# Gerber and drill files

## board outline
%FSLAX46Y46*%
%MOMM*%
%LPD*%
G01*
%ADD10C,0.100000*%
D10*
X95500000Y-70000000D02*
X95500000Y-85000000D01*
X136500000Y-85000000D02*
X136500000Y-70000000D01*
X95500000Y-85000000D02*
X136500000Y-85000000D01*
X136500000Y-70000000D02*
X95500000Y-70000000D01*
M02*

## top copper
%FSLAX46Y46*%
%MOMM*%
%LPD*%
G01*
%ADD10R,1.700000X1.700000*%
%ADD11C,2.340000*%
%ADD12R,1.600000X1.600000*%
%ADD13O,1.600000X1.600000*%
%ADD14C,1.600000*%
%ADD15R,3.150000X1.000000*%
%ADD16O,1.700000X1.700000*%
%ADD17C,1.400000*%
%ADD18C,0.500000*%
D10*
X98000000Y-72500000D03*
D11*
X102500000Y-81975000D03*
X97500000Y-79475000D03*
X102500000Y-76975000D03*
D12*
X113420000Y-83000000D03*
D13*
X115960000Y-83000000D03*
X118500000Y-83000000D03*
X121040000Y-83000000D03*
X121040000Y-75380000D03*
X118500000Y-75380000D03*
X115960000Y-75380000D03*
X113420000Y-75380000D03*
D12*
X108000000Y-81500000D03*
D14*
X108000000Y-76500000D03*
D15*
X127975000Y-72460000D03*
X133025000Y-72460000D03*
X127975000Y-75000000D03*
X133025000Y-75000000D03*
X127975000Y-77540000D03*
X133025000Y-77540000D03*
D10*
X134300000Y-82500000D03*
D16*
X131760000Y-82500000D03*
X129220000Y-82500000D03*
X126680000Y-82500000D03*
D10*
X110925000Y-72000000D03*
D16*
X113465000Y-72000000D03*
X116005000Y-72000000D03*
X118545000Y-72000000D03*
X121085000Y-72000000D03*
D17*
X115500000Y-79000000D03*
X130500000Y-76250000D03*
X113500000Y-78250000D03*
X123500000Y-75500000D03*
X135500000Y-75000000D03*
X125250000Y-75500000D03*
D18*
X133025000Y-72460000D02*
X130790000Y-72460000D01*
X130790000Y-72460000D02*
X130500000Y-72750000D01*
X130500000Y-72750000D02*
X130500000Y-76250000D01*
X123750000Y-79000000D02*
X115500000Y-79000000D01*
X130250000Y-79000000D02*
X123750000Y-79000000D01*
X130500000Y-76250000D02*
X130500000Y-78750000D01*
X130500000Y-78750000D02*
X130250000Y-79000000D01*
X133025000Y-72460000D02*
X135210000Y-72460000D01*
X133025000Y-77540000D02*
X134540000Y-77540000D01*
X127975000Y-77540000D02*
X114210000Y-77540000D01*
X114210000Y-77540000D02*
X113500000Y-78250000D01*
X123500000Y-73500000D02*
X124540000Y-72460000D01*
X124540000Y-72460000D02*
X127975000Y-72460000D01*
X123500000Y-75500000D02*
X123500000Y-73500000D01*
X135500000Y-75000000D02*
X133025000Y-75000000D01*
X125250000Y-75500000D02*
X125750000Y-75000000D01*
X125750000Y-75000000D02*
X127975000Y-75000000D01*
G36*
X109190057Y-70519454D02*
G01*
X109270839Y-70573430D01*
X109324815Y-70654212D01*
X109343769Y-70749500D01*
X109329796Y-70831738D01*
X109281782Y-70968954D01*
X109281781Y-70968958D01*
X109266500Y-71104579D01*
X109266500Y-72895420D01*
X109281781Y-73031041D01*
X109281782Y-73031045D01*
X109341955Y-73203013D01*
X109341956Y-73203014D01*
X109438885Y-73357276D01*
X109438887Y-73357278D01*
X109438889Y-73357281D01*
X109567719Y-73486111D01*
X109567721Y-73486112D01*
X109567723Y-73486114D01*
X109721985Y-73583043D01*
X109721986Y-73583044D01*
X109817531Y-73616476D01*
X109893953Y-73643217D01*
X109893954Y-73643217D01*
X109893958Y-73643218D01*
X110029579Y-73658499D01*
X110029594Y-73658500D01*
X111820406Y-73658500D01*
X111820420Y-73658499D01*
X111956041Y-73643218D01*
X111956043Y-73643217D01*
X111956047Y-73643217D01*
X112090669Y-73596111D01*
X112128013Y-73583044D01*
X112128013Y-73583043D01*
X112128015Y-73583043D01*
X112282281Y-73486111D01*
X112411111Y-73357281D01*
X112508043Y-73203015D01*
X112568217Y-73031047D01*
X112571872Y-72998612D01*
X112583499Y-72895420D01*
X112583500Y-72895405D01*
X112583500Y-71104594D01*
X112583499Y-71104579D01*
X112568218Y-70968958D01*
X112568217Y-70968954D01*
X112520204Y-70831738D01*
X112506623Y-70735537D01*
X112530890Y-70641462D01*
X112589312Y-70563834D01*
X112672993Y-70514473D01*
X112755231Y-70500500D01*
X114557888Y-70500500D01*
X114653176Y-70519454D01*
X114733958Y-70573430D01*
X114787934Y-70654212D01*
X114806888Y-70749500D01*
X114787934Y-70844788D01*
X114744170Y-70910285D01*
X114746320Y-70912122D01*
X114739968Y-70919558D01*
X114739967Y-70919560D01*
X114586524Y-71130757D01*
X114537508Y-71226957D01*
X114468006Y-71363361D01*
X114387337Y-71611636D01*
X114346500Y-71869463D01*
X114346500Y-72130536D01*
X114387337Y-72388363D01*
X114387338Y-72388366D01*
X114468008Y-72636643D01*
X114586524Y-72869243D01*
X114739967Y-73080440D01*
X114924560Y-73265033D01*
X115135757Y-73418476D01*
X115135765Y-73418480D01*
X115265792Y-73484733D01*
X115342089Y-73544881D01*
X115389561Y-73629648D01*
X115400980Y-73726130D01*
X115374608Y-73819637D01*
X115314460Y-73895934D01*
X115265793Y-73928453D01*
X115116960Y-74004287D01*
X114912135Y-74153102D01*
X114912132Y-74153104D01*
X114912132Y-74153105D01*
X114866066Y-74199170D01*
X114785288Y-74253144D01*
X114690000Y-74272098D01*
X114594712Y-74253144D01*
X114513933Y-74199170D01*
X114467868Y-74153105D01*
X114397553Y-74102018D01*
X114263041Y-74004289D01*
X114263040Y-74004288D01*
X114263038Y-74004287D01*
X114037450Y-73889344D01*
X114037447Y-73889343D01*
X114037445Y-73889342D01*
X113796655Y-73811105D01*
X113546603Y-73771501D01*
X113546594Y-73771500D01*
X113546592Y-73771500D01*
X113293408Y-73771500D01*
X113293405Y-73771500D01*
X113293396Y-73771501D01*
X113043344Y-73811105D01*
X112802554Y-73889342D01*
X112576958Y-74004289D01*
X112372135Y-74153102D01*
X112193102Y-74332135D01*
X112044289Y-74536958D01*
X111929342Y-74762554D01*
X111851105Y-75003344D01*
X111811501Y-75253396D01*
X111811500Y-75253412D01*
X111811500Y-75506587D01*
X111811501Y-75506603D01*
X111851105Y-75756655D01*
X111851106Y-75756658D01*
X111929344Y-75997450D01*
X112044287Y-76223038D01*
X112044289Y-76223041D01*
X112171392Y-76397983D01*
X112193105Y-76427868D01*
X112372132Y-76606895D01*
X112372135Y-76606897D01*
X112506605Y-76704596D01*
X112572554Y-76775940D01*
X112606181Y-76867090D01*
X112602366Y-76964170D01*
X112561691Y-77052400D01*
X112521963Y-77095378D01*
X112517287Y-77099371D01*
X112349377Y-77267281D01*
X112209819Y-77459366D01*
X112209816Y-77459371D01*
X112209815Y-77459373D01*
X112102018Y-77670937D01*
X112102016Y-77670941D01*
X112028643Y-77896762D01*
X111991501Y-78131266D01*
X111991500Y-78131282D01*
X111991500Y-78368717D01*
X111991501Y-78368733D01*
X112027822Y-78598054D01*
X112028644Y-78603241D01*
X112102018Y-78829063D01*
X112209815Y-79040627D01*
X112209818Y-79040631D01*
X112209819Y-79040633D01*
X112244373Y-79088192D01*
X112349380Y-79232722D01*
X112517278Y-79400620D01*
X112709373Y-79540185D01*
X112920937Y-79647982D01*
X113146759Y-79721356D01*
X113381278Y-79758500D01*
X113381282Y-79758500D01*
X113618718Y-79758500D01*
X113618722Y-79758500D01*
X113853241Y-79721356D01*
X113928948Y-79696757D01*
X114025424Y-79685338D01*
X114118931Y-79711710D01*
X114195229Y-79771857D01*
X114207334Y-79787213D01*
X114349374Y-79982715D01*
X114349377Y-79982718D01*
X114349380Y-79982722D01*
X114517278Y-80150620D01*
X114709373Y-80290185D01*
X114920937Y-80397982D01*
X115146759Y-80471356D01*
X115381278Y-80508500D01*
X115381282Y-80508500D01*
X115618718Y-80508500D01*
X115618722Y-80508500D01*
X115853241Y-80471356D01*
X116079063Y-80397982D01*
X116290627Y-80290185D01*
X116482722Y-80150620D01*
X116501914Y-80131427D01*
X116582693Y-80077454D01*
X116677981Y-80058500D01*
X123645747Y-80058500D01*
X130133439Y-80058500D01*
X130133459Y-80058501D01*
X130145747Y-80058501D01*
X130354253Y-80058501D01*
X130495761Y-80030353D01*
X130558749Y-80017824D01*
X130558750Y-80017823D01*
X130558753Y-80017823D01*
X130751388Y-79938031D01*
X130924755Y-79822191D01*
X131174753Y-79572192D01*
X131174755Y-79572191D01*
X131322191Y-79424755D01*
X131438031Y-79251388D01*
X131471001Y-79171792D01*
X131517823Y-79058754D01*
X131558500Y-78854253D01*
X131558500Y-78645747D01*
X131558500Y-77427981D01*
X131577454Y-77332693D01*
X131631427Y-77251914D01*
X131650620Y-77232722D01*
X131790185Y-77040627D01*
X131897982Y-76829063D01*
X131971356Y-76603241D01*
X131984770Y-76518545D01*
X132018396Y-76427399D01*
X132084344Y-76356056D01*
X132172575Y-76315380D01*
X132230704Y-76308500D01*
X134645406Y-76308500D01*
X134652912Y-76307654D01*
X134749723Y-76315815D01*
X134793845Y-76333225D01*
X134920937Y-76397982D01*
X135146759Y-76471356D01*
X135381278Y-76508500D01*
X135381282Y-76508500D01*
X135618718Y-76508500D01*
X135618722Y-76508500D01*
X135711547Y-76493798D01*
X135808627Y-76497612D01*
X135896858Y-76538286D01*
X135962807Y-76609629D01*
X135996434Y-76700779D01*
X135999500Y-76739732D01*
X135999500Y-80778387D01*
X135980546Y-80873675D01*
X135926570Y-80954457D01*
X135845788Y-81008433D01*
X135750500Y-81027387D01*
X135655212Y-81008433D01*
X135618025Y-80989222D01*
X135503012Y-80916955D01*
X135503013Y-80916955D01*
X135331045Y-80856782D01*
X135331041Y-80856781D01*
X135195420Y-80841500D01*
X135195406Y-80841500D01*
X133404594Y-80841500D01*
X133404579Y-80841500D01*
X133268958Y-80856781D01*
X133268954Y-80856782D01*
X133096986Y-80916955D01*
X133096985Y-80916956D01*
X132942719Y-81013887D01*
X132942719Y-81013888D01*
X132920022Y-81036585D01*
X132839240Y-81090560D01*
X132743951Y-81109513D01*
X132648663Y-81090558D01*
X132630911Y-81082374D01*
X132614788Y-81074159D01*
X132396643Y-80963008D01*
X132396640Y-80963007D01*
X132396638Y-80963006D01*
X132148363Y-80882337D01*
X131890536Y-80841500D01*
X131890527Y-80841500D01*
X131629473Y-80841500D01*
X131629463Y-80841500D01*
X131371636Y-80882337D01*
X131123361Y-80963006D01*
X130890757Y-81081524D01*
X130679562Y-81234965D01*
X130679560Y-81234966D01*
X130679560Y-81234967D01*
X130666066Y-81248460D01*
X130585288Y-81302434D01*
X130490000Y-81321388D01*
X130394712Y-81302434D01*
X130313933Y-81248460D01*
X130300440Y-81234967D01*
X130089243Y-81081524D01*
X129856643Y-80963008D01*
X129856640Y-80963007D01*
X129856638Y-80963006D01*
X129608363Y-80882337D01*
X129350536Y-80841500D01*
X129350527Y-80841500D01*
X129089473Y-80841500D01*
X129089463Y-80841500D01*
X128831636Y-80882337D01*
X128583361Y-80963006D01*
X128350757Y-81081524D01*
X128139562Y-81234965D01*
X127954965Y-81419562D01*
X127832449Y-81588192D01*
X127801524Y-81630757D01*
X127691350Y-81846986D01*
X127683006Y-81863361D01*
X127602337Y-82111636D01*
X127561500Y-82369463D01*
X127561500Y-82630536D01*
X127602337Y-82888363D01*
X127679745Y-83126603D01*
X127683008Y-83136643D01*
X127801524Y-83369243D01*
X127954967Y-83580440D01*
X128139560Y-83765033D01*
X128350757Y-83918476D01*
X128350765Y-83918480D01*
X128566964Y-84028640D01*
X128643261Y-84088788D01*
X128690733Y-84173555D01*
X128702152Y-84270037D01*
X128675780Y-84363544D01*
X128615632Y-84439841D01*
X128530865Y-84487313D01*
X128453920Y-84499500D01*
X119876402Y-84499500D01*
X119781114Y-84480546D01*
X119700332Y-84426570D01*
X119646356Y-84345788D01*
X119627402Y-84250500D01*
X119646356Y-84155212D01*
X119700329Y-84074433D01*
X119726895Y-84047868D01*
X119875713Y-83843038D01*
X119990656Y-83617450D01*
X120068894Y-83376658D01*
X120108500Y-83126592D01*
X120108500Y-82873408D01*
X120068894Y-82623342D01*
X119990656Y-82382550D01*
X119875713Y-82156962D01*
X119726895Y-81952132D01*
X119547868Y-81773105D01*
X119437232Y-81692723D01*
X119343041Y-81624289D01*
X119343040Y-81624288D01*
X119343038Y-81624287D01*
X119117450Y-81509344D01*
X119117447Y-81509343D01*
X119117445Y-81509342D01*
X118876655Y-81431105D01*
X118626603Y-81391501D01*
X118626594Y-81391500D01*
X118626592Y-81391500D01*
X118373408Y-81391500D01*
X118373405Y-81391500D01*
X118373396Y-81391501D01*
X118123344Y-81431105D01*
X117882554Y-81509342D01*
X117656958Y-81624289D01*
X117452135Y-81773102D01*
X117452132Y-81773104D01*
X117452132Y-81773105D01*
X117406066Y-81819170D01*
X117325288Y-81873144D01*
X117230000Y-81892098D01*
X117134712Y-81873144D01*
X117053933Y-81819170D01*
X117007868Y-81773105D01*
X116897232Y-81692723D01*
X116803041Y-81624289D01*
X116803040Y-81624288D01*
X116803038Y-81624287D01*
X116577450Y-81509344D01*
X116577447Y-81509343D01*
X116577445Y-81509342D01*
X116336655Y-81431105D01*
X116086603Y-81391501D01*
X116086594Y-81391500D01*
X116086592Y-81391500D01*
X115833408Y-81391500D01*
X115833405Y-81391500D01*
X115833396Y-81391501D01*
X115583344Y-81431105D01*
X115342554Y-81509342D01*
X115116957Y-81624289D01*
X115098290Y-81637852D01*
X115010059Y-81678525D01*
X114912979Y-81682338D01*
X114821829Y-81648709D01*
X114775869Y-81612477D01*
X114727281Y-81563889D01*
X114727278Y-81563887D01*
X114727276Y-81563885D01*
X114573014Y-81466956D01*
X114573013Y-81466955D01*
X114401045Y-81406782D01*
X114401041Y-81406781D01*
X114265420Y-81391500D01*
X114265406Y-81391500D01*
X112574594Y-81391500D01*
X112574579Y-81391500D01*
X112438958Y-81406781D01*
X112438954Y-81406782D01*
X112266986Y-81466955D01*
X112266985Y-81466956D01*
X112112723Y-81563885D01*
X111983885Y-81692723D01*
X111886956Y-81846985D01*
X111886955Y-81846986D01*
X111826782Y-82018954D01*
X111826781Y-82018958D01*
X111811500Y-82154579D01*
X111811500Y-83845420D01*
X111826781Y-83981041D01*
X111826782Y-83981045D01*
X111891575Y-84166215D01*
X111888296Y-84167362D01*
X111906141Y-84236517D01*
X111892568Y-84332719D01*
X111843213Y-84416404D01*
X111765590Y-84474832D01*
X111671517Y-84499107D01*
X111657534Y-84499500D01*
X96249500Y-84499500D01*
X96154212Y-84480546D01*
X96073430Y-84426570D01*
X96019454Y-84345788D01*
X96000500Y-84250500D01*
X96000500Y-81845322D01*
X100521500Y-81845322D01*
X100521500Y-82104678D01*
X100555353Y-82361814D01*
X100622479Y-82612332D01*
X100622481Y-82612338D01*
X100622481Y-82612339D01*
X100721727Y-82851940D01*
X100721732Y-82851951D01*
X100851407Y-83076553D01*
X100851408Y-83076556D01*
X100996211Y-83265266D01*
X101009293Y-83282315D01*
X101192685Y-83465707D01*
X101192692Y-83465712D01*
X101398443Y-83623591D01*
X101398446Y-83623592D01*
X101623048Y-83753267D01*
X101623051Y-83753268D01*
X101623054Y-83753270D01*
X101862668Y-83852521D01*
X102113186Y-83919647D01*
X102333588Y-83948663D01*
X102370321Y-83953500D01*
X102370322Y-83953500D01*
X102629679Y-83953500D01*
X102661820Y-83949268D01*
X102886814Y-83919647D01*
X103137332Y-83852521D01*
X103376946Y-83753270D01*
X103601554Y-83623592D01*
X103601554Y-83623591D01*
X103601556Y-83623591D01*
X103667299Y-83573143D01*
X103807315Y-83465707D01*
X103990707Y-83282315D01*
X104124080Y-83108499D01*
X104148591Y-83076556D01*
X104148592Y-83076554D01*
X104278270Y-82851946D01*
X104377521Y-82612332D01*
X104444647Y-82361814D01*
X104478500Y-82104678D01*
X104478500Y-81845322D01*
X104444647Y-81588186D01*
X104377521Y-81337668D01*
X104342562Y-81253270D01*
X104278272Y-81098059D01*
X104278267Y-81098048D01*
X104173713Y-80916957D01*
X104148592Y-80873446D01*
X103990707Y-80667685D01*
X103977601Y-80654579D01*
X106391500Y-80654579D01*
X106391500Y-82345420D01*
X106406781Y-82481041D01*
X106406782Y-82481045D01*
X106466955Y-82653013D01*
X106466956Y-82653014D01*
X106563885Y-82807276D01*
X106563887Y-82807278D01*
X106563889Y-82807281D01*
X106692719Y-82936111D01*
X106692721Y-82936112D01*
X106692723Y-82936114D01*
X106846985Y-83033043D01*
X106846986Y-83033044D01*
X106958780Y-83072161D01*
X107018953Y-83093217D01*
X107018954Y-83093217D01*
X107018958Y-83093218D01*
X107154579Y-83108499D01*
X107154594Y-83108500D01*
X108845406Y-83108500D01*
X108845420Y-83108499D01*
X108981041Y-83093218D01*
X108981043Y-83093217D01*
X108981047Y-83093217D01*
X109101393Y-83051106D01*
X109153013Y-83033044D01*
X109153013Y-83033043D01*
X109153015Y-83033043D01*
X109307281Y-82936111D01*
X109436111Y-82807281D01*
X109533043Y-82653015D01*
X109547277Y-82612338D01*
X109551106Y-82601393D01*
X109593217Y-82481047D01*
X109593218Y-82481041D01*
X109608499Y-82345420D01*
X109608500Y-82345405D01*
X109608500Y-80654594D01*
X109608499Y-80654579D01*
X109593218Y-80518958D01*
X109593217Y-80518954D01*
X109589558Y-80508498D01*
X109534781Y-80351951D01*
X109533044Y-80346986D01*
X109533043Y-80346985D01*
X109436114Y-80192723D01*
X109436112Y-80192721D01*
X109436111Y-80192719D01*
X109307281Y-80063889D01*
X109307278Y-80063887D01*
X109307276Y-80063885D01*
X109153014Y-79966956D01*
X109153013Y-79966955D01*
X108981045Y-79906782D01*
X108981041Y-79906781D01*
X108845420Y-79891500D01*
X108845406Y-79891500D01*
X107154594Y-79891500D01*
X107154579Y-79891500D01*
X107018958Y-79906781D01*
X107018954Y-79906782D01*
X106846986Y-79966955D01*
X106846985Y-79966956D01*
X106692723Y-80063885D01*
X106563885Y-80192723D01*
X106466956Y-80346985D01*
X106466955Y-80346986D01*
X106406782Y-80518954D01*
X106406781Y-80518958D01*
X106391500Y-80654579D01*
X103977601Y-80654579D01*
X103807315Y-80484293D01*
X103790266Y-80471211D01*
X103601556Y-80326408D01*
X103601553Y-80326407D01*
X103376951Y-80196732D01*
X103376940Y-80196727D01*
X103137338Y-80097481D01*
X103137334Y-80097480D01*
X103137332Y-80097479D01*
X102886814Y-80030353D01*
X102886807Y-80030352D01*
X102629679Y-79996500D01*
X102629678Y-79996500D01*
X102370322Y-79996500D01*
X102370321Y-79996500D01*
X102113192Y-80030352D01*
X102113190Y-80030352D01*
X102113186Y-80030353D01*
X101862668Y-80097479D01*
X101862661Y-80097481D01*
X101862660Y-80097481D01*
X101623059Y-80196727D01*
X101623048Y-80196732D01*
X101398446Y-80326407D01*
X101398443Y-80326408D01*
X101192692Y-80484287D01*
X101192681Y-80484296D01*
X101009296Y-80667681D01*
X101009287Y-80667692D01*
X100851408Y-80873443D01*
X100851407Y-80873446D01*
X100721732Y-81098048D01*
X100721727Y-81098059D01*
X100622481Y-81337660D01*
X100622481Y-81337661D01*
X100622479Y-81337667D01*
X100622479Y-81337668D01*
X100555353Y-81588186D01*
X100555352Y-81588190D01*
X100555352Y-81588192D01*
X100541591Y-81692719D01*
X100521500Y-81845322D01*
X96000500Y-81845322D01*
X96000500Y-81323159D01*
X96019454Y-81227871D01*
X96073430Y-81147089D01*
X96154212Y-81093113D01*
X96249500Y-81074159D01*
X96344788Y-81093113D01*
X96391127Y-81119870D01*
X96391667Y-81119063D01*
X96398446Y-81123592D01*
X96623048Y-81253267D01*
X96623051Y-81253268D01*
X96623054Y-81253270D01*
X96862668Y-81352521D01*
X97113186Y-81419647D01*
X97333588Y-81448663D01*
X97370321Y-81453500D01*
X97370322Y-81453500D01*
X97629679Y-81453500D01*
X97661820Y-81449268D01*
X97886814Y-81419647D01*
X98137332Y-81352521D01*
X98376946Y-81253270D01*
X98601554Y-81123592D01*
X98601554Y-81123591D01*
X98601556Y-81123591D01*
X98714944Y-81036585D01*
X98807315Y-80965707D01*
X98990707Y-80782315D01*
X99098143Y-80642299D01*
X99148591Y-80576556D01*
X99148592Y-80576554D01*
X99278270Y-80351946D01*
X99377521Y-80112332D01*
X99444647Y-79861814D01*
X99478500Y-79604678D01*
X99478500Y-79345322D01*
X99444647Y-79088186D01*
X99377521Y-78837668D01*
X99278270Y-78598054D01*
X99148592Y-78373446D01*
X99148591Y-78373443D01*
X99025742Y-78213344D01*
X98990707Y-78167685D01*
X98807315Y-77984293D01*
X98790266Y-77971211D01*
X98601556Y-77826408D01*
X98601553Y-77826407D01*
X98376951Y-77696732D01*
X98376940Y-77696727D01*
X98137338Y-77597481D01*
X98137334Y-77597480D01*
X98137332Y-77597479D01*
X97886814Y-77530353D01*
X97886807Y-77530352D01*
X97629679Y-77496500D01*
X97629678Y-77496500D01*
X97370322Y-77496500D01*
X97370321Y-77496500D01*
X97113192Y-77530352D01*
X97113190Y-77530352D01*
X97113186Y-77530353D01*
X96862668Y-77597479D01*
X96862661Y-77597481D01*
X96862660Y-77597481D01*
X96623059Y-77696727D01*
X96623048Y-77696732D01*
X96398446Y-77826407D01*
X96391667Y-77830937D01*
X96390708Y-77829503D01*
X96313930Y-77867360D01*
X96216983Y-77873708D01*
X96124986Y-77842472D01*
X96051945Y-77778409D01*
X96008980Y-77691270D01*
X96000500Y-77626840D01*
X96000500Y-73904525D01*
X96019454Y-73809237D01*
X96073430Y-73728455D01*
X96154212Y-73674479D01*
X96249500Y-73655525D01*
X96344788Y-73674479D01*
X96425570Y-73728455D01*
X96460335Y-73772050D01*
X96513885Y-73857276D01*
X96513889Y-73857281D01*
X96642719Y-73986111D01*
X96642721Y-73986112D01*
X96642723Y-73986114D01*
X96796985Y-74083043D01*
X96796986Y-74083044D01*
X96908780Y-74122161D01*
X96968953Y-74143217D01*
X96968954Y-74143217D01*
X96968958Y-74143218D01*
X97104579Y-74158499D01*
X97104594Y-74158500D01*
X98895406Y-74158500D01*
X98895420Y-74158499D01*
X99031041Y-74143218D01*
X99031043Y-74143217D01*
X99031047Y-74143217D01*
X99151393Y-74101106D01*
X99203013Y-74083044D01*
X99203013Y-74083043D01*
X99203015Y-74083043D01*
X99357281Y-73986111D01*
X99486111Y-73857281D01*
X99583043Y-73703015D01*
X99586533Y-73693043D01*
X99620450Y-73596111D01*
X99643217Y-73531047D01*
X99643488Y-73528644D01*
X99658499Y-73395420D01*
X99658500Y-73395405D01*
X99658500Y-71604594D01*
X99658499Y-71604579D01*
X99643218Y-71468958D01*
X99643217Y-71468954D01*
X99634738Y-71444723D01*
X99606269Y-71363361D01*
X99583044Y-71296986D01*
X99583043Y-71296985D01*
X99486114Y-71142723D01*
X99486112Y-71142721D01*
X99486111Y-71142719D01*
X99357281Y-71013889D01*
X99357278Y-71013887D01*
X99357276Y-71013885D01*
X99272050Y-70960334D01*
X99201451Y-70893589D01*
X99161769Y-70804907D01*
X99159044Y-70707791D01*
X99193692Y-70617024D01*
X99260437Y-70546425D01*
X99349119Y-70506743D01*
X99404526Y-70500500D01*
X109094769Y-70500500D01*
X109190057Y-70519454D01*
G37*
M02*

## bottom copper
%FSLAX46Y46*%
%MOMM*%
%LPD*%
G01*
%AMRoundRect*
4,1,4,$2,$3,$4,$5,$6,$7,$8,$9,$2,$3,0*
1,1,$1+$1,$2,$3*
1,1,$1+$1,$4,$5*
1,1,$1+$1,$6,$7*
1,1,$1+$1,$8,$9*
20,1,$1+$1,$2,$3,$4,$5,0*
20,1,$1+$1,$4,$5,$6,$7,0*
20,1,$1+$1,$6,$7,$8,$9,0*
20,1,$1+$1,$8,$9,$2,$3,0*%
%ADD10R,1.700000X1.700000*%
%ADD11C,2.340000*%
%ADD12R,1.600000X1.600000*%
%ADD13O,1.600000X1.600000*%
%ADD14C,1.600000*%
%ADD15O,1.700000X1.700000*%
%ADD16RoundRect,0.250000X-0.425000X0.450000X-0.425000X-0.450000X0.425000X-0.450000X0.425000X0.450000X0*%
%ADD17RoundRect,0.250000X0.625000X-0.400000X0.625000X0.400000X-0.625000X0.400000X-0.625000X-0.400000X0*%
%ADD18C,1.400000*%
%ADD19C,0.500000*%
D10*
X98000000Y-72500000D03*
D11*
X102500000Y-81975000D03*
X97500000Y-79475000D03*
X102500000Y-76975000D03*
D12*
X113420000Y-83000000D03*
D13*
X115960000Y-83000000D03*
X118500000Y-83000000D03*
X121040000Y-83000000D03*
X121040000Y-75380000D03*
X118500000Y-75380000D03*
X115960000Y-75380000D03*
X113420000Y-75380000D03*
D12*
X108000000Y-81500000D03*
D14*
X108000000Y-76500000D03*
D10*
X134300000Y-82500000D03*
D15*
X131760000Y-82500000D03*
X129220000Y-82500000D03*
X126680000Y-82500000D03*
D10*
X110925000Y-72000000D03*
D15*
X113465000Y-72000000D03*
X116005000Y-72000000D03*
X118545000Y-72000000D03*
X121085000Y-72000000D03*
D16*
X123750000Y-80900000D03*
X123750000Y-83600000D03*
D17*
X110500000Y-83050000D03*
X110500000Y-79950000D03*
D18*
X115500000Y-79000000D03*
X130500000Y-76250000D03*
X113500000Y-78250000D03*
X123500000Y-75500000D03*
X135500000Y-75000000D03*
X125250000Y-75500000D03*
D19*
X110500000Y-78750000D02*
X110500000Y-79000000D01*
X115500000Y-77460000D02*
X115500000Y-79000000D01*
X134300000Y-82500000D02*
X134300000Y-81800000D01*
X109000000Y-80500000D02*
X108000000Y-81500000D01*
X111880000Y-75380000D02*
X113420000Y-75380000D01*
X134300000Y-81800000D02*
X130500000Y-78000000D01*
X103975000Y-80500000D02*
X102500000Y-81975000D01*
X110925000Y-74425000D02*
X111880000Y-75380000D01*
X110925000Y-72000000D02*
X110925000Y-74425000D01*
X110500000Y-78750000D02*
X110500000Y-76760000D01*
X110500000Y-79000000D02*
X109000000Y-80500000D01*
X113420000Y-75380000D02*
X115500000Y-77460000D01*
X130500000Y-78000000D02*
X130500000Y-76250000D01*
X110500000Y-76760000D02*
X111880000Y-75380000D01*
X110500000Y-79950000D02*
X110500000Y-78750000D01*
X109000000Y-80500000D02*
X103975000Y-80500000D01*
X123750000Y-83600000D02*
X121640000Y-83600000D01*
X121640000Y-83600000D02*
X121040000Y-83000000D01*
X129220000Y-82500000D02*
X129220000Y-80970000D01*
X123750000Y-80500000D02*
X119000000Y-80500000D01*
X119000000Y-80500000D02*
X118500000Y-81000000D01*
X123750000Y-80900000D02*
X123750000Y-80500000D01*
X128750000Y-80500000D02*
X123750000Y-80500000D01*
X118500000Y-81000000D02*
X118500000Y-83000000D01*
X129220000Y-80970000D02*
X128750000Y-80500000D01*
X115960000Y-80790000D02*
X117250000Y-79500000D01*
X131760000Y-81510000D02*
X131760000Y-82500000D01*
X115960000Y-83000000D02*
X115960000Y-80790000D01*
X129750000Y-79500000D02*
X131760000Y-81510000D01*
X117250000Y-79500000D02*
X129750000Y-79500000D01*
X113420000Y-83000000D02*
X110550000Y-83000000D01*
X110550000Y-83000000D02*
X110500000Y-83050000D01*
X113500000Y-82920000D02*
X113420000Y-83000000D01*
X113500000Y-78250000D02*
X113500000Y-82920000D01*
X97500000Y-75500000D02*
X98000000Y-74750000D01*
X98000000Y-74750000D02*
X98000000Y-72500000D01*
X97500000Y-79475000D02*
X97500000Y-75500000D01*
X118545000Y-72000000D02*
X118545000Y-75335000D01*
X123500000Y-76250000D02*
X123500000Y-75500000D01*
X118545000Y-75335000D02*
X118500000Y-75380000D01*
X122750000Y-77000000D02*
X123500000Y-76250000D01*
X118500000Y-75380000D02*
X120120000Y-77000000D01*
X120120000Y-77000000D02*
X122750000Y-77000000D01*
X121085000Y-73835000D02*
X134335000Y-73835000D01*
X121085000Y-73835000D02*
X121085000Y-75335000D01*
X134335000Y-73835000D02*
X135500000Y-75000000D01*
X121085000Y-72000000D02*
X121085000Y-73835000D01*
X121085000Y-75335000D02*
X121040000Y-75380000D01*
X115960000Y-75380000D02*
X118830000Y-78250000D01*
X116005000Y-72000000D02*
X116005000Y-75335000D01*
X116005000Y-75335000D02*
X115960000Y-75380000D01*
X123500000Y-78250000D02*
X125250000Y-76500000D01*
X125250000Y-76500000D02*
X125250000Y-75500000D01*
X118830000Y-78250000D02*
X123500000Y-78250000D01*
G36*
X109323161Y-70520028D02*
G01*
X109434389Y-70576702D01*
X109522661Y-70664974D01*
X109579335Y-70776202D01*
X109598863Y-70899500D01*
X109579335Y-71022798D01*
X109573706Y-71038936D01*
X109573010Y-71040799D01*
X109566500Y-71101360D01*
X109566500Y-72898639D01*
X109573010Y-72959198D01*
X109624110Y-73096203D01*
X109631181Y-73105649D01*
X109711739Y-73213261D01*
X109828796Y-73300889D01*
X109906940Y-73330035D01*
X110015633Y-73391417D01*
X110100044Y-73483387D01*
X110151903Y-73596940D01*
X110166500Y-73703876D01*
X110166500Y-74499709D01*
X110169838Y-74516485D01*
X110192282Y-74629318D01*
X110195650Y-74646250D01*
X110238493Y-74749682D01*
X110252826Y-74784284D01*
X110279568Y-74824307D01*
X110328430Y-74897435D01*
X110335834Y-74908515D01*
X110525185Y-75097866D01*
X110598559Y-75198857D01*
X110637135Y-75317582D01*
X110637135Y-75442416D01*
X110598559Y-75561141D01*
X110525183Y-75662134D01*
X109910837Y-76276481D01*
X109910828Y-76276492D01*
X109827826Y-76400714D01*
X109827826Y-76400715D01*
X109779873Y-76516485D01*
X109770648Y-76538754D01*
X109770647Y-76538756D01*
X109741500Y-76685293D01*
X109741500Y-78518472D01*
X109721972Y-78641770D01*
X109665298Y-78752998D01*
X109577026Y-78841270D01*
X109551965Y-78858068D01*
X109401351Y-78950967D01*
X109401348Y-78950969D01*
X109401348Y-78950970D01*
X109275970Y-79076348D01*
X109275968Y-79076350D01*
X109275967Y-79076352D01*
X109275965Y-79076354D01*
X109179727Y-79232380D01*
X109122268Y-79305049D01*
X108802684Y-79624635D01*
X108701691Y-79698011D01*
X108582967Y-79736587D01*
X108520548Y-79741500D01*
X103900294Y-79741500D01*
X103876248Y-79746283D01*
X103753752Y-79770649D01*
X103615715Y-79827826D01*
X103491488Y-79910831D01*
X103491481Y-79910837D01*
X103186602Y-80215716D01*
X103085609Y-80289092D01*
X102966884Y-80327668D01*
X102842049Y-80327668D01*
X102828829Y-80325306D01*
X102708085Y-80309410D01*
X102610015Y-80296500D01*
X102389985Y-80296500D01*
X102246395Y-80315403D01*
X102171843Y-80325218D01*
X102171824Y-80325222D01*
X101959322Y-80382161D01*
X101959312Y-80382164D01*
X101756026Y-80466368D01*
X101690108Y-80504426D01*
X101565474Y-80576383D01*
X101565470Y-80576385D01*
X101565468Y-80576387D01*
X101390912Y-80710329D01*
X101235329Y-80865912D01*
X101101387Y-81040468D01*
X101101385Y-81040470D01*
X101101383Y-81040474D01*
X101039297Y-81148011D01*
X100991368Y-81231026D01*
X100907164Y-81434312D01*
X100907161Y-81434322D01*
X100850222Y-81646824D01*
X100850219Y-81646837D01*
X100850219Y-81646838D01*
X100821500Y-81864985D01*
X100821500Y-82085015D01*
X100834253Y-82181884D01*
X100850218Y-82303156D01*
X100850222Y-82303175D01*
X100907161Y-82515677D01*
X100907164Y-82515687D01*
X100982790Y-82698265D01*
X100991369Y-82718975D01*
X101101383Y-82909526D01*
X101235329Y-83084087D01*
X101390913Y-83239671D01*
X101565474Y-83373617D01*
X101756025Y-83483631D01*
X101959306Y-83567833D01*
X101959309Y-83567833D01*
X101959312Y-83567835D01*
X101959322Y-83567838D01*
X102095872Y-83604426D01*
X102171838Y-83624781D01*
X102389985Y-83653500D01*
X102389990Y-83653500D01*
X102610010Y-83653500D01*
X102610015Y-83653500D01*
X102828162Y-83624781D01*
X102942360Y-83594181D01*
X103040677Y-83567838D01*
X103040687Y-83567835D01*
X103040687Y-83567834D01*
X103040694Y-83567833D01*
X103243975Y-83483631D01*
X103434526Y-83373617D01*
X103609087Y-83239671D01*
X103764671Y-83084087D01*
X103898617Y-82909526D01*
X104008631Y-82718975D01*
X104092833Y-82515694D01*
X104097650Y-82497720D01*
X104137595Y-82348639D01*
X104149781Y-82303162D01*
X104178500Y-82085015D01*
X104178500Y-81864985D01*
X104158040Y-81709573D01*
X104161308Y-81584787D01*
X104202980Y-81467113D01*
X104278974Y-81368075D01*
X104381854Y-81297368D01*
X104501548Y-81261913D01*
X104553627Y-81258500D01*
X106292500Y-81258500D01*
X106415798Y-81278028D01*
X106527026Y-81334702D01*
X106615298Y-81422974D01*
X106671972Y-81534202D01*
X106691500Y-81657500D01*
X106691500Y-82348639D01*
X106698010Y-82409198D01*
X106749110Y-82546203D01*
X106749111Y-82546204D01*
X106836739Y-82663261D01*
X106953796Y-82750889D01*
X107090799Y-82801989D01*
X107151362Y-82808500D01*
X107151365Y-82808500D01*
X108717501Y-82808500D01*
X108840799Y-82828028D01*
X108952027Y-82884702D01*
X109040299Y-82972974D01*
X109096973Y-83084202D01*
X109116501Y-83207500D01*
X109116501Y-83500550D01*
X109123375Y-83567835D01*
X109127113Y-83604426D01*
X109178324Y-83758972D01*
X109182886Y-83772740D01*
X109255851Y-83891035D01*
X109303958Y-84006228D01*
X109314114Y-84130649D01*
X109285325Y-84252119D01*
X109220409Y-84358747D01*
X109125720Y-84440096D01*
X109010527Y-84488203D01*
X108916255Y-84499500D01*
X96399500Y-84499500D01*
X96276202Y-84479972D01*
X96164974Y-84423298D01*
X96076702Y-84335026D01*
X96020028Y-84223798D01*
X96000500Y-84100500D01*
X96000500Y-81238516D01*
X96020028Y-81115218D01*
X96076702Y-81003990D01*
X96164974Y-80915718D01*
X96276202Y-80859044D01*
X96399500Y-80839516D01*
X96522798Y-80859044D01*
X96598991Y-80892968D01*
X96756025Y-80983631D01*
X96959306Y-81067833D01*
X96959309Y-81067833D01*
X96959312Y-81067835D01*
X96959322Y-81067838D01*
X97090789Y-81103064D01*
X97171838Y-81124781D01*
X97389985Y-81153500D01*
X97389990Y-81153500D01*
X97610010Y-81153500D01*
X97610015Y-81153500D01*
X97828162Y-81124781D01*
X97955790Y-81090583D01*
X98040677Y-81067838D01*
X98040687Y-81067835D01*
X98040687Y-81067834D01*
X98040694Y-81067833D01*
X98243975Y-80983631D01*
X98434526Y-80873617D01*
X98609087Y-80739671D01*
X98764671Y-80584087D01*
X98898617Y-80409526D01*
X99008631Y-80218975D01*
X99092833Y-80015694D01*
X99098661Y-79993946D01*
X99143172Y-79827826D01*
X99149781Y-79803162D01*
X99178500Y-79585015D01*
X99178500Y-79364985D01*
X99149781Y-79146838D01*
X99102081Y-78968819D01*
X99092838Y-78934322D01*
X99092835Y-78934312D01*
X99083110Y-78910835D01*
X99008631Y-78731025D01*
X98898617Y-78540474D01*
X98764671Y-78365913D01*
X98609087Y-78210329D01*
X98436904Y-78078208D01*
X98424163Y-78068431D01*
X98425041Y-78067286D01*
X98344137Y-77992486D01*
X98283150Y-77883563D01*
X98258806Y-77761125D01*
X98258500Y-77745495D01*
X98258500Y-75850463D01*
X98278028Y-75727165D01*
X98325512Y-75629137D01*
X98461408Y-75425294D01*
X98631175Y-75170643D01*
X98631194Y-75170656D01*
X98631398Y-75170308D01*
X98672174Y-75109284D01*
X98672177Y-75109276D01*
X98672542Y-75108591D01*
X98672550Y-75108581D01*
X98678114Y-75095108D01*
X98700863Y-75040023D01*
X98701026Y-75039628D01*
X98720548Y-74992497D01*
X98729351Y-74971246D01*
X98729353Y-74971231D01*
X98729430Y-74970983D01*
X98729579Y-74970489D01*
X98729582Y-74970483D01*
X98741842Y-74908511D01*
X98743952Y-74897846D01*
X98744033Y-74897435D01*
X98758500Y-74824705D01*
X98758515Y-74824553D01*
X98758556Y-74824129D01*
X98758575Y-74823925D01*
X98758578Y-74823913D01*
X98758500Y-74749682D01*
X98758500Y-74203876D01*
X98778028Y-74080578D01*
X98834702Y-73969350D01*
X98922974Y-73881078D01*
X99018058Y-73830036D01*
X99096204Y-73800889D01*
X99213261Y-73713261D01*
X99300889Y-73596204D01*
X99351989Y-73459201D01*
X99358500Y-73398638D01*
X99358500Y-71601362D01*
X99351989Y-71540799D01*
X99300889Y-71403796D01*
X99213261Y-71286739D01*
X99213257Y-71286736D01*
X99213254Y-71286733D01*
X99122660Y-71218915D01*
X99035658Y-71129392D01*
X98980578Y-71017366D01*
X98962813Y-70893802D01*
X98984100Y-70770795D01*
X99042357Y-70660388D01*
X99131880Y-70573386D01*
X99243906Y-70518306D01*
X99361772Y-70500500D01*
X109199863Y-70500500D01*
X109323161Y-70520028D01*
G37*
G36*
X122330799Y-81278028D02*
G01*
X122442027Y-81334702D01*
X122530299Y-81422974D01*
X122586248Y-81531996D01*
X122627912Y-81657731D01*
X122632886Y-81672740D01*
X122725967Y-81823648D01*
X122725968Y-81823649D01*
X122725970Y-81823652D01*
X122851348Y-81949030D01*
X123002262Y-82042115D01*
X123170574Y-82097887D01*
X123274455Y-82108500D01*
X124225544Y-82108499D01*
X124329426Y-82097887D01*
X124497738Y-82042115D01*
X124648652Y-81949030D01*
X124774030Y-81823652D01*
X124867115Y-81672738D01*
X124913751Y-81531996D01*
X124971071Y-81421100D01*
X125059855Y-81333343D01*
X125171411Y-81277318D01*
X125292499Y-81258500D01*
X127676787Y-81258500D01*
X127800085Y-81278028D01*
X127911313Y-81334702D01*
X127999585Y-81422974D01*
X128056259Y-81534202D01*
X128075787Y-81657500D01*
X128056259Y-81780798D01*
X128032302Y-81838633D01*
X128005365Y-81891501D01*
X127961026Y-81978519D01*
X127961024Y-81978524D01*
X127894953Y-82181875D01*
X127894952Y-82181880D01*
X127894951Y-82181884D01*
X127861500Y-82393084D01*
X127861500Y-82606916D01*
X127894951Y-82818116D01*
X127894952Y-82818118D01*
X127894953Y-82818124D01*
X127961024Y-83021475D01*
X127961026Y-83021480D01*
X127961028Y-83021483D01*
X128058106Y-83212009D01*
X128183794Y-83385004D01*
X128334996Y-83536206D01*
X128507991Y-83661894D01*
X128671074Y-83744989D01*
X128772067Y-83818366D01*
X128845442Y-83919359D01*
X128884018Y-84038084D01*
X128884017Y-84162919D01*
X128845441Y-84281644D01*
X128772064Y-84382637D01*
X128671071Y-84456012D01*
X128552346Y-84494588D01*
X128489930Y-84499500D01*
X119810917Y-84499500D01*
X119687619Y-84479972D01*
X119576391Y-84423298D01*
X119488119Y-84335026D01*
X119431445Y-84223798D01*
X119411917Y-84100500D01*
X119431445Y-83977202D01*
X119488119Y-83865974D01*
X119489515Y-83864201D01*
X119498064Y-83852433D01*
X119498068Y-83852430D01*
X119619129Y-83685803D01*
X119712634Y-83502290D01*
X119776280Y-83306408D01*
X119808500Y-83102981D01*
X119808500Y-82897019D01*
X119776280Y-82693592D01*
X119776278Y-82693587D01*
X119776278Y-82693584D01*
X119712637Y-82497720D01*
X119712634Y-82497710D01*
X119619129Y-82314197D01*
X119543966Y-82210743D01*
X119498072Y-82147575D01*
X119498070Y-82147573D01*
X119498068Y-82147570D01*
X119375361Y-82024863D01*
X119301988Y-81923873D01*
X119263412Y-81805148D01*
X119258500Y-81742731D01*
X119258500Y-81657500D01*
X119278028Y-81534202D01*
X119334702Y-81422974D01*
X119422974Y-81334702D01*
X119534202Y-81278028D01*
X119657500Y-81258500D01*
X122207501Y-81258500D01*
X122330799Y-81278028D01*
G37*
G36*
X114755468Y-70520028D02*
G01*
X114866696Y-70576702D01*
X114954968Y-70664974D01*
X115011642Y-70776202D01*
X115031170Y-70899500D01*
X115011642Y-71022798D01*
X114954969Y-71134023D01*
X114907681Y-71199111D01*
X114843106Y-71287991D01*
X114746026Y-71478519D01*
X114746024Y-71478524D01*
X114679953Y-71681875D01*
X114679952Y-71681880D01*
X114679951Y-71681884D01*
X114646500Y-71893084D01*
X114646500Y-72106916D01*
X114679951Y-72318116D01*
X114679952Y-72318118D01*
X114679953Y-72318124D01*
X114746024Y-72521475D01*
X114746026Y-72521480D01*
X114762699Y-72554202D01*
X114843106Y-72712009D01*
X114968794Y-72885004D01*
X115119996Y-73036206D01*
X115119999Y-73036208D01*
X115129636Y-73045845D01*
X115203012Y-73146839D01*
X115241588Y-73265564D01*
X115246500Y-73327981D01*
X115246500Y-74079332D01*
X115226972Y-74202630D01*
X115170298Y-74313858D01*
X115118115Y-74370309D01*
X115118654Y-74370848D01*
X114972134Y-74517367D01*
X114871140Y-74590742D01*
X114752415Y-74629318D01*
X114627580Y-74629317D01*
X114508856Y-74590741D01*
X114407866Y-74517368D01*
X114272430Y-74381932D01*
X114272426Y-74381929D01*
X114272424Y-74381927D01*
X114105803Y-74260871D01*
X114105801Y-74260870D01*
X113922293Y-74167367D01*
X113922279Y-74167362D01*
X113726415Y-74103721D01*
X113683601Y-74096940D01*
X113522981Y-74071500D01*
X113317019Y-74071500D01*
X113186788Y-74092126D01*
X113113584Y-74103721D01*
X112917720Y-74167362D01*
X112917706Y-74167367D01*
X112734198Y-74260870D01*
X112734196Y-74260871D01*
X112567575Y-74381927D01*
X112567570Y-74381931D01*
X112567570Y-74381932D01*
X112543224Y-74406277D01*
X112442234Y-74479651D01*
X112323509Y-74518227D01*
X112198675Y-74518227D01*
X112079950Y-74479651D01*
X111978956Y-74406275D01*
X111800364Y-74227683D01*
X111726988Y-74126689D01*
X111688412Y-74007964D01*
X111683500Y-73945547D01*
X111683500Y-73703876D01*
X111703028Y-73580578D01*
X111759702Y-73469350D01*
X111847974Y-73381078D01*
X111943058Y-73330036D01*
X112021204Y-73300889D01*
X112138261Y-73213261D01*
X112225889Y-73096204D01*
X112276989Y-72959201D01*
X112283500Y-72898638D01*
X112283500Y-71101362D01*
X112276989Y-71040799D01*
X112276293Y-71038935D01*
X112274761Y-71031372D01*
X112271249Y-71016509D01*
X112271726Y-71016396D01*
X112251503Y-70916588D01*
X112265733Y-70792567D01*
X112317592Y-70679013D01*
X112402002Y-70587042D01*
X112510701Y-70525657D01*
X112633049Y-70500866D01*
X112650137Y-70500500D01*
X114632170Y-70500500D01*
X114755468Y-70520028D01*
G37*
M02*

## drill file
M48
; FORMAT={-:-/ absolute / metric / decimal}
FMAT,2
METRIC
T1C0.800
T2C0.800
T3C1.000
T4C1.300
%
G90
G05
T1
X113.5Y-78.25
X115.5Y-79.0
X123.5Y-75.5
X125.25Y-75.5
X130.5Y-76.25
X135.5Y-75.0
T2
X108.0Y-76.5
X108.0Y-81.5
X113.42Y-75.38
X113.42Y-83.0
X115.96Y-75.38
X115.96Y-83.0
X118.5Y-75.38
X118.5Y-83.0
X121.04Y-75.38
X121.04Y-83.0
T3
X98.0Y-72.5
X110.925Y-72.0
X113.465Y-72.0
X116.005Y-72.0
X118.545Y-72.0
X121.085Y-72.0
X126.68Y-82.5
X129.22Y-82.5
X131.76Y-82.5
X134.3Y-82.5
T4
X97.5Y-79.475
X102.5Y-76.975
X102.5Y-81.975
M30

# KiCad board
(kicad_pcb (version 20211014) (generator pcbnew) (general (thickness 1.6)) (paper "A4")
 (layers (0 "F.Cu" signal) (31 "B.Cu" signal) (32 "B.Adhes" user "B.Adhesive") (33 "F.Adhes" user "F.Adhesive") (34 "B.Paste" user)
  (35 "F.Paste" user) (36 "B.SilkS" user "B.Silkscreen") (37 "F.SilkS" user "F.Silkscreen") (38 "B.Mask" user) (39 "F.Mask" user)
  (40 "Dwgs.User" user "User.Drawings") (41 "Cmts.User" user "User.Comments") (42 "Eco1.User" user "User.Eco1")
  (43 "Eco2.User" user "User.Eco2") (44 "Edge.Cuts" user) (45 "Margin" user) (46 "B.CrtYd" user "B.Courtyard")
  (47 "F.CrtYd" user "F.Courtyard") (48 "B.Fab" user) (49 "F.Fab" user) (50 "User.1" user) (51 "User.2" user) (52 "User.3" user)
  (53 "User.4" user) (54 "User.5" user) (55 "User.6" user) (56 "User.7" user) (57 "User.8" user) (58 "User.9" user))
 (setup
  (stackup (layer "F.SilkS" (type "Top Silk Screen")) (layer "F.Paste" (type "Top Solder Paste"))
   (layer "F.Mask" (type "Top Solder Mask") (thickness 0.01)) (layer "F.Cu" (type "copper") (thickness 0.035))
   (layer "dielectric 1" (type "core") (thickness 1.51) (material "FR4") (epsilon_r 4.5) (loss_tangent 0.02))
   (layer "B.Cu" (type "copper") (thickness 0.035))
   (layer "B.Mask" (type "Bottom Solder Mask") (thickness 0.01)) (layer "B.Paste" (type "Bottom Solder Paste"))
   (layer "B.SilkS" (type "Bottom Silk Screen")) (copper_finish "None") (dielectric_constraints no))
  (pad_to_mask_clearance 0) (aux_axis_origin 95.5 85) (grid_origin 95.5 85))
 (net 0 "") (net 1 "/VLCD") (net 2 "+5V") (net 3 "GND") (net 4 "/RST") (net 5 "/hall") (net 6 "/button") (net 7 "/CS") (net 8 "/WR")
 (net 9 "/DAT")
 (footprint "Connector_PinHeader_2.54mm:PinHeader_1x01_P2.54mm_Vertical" (layer "F.Cu") (at 98 72.5)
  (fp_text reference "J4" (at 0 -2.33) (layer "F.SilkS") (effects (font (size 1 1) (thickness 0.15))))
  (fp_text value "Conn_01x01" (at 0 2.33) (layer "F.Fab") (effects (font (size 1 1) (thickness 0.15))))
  (pad "1" thru_hole rect (at 0 0) (size 1.7 1.7) (drill 1) (layers *.Cu *.Mask) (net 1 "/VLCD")))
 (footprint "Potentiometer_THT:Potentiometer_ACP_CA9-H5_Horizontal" (layer "F.Cu") (at 102.5 81.975 180)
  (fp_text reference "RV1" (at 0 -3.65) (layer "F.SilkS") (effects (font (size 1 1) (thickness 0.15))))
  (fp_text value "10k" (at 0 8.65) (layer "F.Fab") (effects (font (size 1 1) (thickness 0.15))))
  (pad "1" thru_hole circle (at 0 0 180) (size 2.34 2.34) (drill 1.3) (layers *.Cu *.Mask) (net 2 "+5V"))
  (pad "2" thru_hole circle (at 5 2.5 180) (size 2.34 2.34) (drill 1.3) (layers *.Cu *.Mask) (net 1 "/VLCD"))
  (pad "3" thru_hole circle (at 0 5 180) (size 2.34 2.34) (drill 1.3) (layers *.Cu *.Mask) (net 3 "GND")))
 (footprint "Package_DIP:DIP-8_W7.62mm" (layer "F.Cu") (at 113.42 83 90)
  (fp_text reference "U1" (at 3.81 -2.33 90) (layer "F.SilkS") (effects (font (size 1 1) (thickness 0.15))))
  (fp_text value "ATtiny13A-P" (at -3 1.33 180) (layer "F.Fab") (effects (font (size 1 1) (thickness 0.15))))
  (pad "1" thru_hole rect (at 0 0 90) (size 1.6 1.6) (drill 0.8) (layers *.Cu *.Mask) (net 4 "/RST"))
  (pad "2" thru_hole oval (at 0 2.54 90) (size 1.6 1.6) (drill 0.8) (layers *.Cu *.Mask) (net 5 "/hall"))
  (pad "3" thru_hole oval (at 0 5.08 90) (size 1.6 1.6) (drill 0.8) (layers *.Cu *.Mask) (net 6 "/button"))
  (pad "4" thru_hole oval (at 0 7.62 90) (size 1.6 1.6) (drill 0.8) (layers *.Cu *.Mask) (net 3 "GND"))
  (pad "5" thru_hole oval (at 7.62 7.62 90) (size 1.6 1.6) (drill 0.8) (layers *.Cu *.Mask) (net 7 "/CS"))
  (pad "6" thru_hole oval (at 7.62 5.08 90) (size 1.6 1.6) (drill 0.8) (layers *.Cu *.Mask) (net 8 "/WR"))
  (pad "7" thru_hole oval (at 7.62 2.54 90) (size 1.6 1.6) (drill 0.8) (layers *.Cu *.Mask) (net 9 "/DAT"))
  (pad "8" thru_hole oval (at 7.62 0 90) (size 1.6 1.6) (drill 0.8) (layers *.Cu *.Mask) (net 2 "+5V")))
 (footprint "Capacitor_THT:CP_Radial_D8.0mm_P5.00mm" (layer "F.Cu") (at 108 81.5 90)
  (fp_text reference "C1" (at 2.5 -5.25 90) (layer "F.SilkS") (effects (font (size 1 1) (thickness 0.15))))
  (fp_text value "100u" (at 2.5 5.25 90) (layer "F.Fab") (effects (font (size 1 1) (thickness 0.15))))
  (pad "1" thru_hole rect (at 0 0 90) (size 1.6 1.6) (drill 0.8) (layers *.Cu *.Mask) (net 2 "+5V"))
  (pad "2" thru_hole circle (at 5 0 90) (size 1.6 1.6) (drill 0.8) (layers *.Cu *.Mask) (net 3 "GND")))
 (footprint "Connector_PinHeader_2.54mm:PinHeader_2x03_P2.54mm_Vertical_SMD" (layer "F.Cu") (at 130.5 75)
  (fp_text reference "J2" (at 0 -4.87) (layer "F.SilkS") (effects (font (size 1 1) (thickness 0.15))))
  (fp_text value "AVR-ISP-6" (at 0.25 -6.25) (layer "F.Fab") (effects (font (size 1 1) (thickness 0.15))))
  (pad "1" smd rect (at -2.525 -2.54) (size 3.15 1) (layers "F.Cu" "F.Paste" "F.Mask") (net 8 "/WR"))
  (pad "2" smd rect (at 2.525 -2.54) (size 3.15 1) (layers "F.Cu" "F.Paste" "F.Mask") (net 2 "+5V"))
  (pad "3" smd rect (at -2.525 0) (size 3.15 1) (layers "F.Cu" "F.Paste" "F.Mask") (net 9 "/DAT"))
  (pad "4" smd rect (at 2.525 0) (size 3.15 1) (layers "F.Cu" "F.Paste" "F.Mask") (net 7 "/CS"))
  (pad "5" smd rect (at -2.525 2.54) (size 3.15 1) (layers "F.Cu" "F.Paste" "F.Mask") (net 4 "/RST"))
  (pad "6" smd rect (at 2.525 2.54) (size 3.15 1) (layers "F.Cu" "F.Paste" "F.Mask") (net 3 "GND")))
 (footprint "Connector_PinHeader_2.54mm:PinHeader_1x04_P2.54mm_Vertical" (layer "F.Cu") (at 134.3 82.5 -90)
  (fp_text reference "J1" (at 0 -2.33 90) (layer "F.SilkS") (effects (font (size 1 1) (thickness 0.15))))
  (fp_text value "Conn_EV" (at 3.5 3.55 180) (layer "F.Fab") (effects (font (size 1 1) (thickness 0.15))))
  (pad "1" thru_hole rect (at 0 0 270) (size 1.7 1.7) (drill 1) (layers *.Cu *.Mask) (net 2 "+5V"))
  (pad "2" thru_hole oval (at 0 2.54 270) (size 1.7 1.7) (drill 1) (layers *.Cu *.Mask) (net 5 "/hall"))
  (pad "3" thru_hole oval (at 0 5.08 270) (size 1.7 1.7) (drill 1) (layers *.Cu *.Mask) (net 6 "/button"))
  (pad "4" thru_hole oval (at 0 7.62 270) (size 1.7 1.7) (drill 1) (layers *.Cu *.Mask) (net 3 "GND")))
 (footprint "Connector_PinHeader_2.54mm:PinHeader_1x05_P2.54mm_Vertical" (layer "F.Cu") (at 110.925 72 90)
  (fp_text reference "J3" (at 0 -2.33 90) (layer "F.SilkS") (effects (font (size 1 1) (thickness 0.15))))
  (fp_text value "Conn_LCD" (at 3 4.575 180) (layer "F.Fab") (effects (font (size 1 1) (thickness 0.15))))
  (pad "1" thru_hole rect (at 0 0 90) (size 1.7 1.7) (drill 1) (layers *.Cu *.Mask) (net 2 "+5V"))
  (pad "2" thru_hole oval (at 0 2.54 90) (size 1.7 1.7) (drill 1) (layers *.Cu *.Mask) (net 3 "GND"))
  (pad "3" thru_hole oval (at 0 5.08 90) (size 1.7 1.7) (drill 1) (layers *.Cu *.Mask) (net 9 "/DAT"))
  (pad "4" thru_hole oval (at 0 7.62 90) (size 1.7 1.7) (drill 1) (layers *.Cu *.Mask) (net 8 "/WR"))
  (pad "5" thru_hole oval (at 0 10.16 90) (size 1.7 1.7) (drill 1) (layers *.Cu *.Mask) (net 7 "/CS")))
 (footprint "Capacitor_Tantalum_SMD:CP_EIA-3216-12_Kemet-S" (layer "B.Cu") (at 123.75 82.25 -90)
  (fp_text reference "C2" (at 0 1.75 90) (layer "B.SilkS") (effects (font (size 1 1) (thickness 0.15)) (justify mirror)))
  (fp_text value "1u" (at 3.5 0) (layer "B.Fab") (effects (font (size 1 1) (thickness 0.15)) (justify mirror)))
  (pad "1" smd roundrect (at -1.35 0 270) (size 1.4 1.35) (layers "B.Cu" "B.Paste" "B.Mask") (roundrect_rratio 0.1851851852)
   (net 6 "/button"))
  (pad "2" smd roundrect (at 1.35 0 270) (size 1.4 1.35) (layers "B.Cu" "B.Paste" "B.Mask") (roundrect_rratio 0.1851851852) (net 3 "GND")))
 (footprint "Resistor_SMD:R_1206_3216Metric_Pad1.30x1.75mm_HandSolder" (layer "B.Cu") (at 110.5 81.5 90)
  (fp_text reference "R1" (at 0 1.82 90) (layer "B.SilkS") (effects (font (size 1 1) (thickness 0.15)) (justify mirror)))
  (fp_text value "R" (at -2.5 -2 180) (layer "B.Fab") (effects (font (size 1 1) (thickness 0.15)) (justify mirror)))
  (pad "1" smd roundrect (at -1.55 0 90) (size 1.3 1.75) (layers "B.Cu" "B.Paste" "B.Mask") (roundrect_rratio 0.1923076923) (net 4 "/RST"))
  (pad "2" smd roundrect (at 1.55 0 90) (size 1.3 1.75) (layers "B.Cu" "B.Paste" "B.Mask") (roundrect_rratio 0.1923076923) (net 2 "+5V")))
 (gr_line (start 95.5 70) (end 95.5 85) (layer "Edge.Cuts") (width 0.1))
 (gr_line (start 136.5 85) (end 136.5 70) (layer "Edge.Cuts") (width 0.1))
 (gr_line (start 95.5 85) (end 136.5 85) (layer "Edge.Cuts") (width 0.1))
 (gr_line (start 136.5 70) (end 95.5 70) (layer "Edge.Cuts") (width 0.1))
 (segment (start 133.025 72.46) (end 130.79 72.46) (width 0.5) (layer "F.Cu") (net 2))
 (segment (start 130.79 72.46) (end 130.5 72.75) (width 0.5) (layer "F.Cu") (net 2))
 (segment (start 130.5 72.75) (end 130.5 76.25) (width 0.5) (layer "F.Cu") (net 2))
 (segment (start 123.75 79) (end 115.5 79) (width 0.5) (layer "F.Cu") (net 2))
 (segment (start 130.25 79) (end 123.75 79) (width 0.5) (layer "F.Cu") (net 2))
 (segment (start 130.5 76.25) (end 130.5 78.75) (width 0.5) (layer "F.Cu") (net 2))
 (segment (start 130.5 78.75) (end 130.25 79) (width 0.5) (layer "F.Cu") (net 2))
 (segment (start 133.025 72.46) (end 135.21 72.46) (width 0.5) (layer "F.Cu") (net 2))
 (via (at 115.5 79) (size 1.4) (drill 0.8) (layers "F.Cu" "B.Cu") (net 2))
 (via (at 130.5 76.25) (size 1.4) (drill 0.8) (layers "F.Cu" "B.Cu") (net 2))
 (segment (start 110.5 78.75) (end 110.5 79) (width 0.5) (layer "B.Cu") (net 2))
 (segment (start 115.5 77.46) (end 115.5 79) (width 0.5) (layer "B.Cu") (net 2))
 (segment (start 134.3 82.5) (end 134.3 81.8) (width 0.5) (layer "B.Cu") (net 2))
 (segment (start 109 80.5) (end 108 81.5) (width 0.5) (layer "B.Cu") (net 2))
 (segment (start 111.88 75.38) (end 113.42 75.38) (width 0.5) (layer "B.Cu") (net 2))
 (segment (start 134.3 81.8) (end 130.5 78) (width 0.5) (layer "B.Cu") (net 2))
 (segment (start 103.975 80.5) (end 102.5 81.975) (width 0.5) (layer "B.Cu") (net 2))
 (segment (start 110.925 74.425) (end 111.88 75.38) (width 0.5) (layer "B.Cu") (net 2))
 (segment (start 110.925 72) (end 110.925 74.425) (width 0.5) (layer "B.Cu") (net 2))
 (segment (start 110.5 78.75) (end 110.5 76.76) (width 0.5) (layer "B.Cu") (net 2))
 (segment (start 110.5 79) (end 109 80.5) (width 0.5) (layer "B.Cu") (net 2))
 (segment (start 113.42 75.38) (end 115.5 77.46) (width 0.5) (layer "B.Cu") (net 2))
 (segment (start 130.5 78) (end 130.5 76.25) (width 0.5) (layer "B.Cu") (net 2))
 (segment (start 110.5 76.76) (end 111.88 75.38) (width 0.5) (layer "B.Cu") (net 2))
 (segment (start 110.5 79.95) (end 110.5 78.75) (width 0.5) (layer "B.Cu") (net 2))
 (segment (start 109 80.5) (end 103.975 80.5) (width 0.5) (layer "B.Cu") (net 2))
 (segment (start 133.025 77.54) (end 134.54 77.54) (width 0.5) (layer "F.Cu") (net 3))
 (segment (start 123.75 83.6) (end 121.64 83.6) (width 0.5) (layer "B.Cu") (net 3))
 (segment (start 121.64 83.6) (end 121.04 83) (width 0.5) (layer "B.Cu") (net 3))
 (segment (start 129.22 82.5) (end 129.22 80.97) (width 0.5) (layer "B.Cu") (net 6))
 (segment (start 123.75 80.5) (end 119 80.5) (width 0.5) (layer "B.Cu") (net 6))
 (segment (start 119 80.5) (end 118.5 81) (width 0.5) (layer "B.Cu") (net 6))
 (segment (start 123.75 80.9) (end 123.75 80.5) (width 0.5) (layer "B.Cu") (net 6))
 (segment (start 128.75 80.5) (end 123.75 80.5) (width 0.5) (layer "B.Cu") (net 6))
 (segment (start 118.5 81) (end 118.5 83) (width 0.5) (layer "B.Cu") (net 6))
 (segment (start 129.22 80.97) (end 128.75 80.5) (width 0.5) (layer "B.Cu") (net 6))
 (segment (start 115.96 80.79) (end 117.25 79.5) (width 0.5) (layer "B.Cu") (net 5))
 (segment (start 131.76 81.51) (end 131.76 82.5) (width 0.5) (layer "B.Cu") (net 5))
 (segment (start 115.96 83) (end 115.96 80.79) (width 0.5) (layer "B.Cu") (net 5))
 (segment (start 129.75 79.5) (end 131.76 81.51) (width 0.5) (layer "B.Cu") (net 5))
 (segment (start 117.25 79.5) (end 129.75 79.5) (width 0.5) (layer "B.Cu") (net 5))
 (segment (start 127.975 77.54) (end 114.21 77.54) (width 0.5) (layer "F.Cu") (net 4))
 (segment (start 114.21 77.54) (end 113.5 78.25) (width 0.5) (layer "F.Cu") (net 4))
 (via (at 113.5 78.25) (size 1.4) (drill 0.8) (layers "F.Cu" "B.Cu") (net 4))
 (segment (start 113.42 83) (end 110.55 83) (width 0.5) (layer "B.Cu") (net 4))
 (segment (start 110.55 83) (end 110.5 83.05) (width 0.5) (layer "B.Cu") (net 4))
 (segment (start 113.5 82.92) (end 113.42 83) (width 0.5) (layer "B.Cu") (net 4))
 (segment (start 113.5 78.25) (end 113.5 82.92) (width 0.5) (layer "B.Cu") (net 4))
 (segment (start 97.5 75.5) (end 98 74.75) (width 0.5) (layer "B.Cu") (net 1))
 (segment (start 98 74.75) (end 98 72.5) (width 0.5) (layer "B.Cu") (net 1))
 (segment (start 97.5 79.475) (end 97.5 75.5) (width 0.5) (layer "B.Cu") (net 1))
 (segment (start 123.5 73.5) (end 124.54 72.46) (width 0.5) (layer "F.Cu") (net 8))
 (segment (start 124.54 72.46) (end 127.975 72.46) (width 0.5) (layer "F.Cu") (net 8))
 (segment (start 123.5 75.5) (end 123.5 73.5) (width 0.5) (layer "F.Cu") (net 8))
 (via (at 123.5 75.5) (size 1.4) (drill 0.8) (layers "F.Cu" "B.Cu") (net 8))
 (segment (start 118.545 72) (end 118.545 75.335) (width 0.5) (layer "B.Cu") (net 8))
 (segment (start 123.5 76.25) (end 123.5 75.5) (width 0.5) (layer "B.Cu") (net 8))
 (segment (start 118.545 75.335) (end 118.5 75.38) (width 0.5) (layer "B.Cu") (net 8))
 (segment (start 122.75 77) (end 123.5 76.25) (width 0.5) (layer "B.Cu") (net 8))
 (segment (start 118.5 75.38) (end 120.12 77) (width 0.5) (layer "B.Cu") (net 8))
 (segment (start 120.12 77) (end 122.75 77) (width 0.5) (layer "B.Cu") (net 8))
 (segment (start 135.5 75) (end 133.025 75) (width 0.5) (layer "F.Cu") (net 7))
 (via (at 135.5 75) (size 1.4) (drill 0.8) (layers "F.Cu" "B.Cu") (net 7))
 (segment (start 121.085 73.835) (end 134.335 73.835) (width 0.5) (layer "B.Cu") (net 7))
 (segment (start 121.085 73.835) (end 121.085 75.335) (width 0.5) (layer "B.Cu") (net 7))
 (segment (start 134.335 73.835) (end 135.5 75) (width 0.5) (layer "B.Cu") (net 7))
 (segment (start 121.085 72) (end 121.085 73.835) (width 0.5) (layer "B.Cu") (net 7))
 (segment (start 121.085 75.335) (end 121.04 75.38) (width 0.5) (layer "B.Cu") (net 7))
 (segment (start 125.25 75.5) (end 125.75 75) (width 0.5) (layer "F.Cu") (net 9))
 (segment (start 125.75 75) (end 127.975 75) (width 0.5) (layer "F.Cu") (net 9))
 (via (at 125.25 75.5) (size 1.4) (drill 0.8) (layers "F.Cu" "B.Cu") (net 9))
 (segment (start 115.96 75.38) (end 118.83 78.25) (width 0.5) (layer "B.Cu") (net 9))
 (segment (start 116.005 72) (end 116.005 75.335) (width 0.5) (layer "B.Cu") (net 9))
 (segment (start 116.005 75.335) (end 115.96 75.38) (width 0.5) (layer "B.Cu") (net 9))
 (segment (start 123.5 78.25) (end 125.25 76.5) (width 0.5) (layer "B.Cu") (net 9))
 (segment (start 125.25 76.5) (end 125.25 75.5) (width 0.5) (layer "B.Cu") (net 9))
 (segment (start 118.83 78.25) (end 123.5 78.25) (width 0.5) (layer "B.Cu") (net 9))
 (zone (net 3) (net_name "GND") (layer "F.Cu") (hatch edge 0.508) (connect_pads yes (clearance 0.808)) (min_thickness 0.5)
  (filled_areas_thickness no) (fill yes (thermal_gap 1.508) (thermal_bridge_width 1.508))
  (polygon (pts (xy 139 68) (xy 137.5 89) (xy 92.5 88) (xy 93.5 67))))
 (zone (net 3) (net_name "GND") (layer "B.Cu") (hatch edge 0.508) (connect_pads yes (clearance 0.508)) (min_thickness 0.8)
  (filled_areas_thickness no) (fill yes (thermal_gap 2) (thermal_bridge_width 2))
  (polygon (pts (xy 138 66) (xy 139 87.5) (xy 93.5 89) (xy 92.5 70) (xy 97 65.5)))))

